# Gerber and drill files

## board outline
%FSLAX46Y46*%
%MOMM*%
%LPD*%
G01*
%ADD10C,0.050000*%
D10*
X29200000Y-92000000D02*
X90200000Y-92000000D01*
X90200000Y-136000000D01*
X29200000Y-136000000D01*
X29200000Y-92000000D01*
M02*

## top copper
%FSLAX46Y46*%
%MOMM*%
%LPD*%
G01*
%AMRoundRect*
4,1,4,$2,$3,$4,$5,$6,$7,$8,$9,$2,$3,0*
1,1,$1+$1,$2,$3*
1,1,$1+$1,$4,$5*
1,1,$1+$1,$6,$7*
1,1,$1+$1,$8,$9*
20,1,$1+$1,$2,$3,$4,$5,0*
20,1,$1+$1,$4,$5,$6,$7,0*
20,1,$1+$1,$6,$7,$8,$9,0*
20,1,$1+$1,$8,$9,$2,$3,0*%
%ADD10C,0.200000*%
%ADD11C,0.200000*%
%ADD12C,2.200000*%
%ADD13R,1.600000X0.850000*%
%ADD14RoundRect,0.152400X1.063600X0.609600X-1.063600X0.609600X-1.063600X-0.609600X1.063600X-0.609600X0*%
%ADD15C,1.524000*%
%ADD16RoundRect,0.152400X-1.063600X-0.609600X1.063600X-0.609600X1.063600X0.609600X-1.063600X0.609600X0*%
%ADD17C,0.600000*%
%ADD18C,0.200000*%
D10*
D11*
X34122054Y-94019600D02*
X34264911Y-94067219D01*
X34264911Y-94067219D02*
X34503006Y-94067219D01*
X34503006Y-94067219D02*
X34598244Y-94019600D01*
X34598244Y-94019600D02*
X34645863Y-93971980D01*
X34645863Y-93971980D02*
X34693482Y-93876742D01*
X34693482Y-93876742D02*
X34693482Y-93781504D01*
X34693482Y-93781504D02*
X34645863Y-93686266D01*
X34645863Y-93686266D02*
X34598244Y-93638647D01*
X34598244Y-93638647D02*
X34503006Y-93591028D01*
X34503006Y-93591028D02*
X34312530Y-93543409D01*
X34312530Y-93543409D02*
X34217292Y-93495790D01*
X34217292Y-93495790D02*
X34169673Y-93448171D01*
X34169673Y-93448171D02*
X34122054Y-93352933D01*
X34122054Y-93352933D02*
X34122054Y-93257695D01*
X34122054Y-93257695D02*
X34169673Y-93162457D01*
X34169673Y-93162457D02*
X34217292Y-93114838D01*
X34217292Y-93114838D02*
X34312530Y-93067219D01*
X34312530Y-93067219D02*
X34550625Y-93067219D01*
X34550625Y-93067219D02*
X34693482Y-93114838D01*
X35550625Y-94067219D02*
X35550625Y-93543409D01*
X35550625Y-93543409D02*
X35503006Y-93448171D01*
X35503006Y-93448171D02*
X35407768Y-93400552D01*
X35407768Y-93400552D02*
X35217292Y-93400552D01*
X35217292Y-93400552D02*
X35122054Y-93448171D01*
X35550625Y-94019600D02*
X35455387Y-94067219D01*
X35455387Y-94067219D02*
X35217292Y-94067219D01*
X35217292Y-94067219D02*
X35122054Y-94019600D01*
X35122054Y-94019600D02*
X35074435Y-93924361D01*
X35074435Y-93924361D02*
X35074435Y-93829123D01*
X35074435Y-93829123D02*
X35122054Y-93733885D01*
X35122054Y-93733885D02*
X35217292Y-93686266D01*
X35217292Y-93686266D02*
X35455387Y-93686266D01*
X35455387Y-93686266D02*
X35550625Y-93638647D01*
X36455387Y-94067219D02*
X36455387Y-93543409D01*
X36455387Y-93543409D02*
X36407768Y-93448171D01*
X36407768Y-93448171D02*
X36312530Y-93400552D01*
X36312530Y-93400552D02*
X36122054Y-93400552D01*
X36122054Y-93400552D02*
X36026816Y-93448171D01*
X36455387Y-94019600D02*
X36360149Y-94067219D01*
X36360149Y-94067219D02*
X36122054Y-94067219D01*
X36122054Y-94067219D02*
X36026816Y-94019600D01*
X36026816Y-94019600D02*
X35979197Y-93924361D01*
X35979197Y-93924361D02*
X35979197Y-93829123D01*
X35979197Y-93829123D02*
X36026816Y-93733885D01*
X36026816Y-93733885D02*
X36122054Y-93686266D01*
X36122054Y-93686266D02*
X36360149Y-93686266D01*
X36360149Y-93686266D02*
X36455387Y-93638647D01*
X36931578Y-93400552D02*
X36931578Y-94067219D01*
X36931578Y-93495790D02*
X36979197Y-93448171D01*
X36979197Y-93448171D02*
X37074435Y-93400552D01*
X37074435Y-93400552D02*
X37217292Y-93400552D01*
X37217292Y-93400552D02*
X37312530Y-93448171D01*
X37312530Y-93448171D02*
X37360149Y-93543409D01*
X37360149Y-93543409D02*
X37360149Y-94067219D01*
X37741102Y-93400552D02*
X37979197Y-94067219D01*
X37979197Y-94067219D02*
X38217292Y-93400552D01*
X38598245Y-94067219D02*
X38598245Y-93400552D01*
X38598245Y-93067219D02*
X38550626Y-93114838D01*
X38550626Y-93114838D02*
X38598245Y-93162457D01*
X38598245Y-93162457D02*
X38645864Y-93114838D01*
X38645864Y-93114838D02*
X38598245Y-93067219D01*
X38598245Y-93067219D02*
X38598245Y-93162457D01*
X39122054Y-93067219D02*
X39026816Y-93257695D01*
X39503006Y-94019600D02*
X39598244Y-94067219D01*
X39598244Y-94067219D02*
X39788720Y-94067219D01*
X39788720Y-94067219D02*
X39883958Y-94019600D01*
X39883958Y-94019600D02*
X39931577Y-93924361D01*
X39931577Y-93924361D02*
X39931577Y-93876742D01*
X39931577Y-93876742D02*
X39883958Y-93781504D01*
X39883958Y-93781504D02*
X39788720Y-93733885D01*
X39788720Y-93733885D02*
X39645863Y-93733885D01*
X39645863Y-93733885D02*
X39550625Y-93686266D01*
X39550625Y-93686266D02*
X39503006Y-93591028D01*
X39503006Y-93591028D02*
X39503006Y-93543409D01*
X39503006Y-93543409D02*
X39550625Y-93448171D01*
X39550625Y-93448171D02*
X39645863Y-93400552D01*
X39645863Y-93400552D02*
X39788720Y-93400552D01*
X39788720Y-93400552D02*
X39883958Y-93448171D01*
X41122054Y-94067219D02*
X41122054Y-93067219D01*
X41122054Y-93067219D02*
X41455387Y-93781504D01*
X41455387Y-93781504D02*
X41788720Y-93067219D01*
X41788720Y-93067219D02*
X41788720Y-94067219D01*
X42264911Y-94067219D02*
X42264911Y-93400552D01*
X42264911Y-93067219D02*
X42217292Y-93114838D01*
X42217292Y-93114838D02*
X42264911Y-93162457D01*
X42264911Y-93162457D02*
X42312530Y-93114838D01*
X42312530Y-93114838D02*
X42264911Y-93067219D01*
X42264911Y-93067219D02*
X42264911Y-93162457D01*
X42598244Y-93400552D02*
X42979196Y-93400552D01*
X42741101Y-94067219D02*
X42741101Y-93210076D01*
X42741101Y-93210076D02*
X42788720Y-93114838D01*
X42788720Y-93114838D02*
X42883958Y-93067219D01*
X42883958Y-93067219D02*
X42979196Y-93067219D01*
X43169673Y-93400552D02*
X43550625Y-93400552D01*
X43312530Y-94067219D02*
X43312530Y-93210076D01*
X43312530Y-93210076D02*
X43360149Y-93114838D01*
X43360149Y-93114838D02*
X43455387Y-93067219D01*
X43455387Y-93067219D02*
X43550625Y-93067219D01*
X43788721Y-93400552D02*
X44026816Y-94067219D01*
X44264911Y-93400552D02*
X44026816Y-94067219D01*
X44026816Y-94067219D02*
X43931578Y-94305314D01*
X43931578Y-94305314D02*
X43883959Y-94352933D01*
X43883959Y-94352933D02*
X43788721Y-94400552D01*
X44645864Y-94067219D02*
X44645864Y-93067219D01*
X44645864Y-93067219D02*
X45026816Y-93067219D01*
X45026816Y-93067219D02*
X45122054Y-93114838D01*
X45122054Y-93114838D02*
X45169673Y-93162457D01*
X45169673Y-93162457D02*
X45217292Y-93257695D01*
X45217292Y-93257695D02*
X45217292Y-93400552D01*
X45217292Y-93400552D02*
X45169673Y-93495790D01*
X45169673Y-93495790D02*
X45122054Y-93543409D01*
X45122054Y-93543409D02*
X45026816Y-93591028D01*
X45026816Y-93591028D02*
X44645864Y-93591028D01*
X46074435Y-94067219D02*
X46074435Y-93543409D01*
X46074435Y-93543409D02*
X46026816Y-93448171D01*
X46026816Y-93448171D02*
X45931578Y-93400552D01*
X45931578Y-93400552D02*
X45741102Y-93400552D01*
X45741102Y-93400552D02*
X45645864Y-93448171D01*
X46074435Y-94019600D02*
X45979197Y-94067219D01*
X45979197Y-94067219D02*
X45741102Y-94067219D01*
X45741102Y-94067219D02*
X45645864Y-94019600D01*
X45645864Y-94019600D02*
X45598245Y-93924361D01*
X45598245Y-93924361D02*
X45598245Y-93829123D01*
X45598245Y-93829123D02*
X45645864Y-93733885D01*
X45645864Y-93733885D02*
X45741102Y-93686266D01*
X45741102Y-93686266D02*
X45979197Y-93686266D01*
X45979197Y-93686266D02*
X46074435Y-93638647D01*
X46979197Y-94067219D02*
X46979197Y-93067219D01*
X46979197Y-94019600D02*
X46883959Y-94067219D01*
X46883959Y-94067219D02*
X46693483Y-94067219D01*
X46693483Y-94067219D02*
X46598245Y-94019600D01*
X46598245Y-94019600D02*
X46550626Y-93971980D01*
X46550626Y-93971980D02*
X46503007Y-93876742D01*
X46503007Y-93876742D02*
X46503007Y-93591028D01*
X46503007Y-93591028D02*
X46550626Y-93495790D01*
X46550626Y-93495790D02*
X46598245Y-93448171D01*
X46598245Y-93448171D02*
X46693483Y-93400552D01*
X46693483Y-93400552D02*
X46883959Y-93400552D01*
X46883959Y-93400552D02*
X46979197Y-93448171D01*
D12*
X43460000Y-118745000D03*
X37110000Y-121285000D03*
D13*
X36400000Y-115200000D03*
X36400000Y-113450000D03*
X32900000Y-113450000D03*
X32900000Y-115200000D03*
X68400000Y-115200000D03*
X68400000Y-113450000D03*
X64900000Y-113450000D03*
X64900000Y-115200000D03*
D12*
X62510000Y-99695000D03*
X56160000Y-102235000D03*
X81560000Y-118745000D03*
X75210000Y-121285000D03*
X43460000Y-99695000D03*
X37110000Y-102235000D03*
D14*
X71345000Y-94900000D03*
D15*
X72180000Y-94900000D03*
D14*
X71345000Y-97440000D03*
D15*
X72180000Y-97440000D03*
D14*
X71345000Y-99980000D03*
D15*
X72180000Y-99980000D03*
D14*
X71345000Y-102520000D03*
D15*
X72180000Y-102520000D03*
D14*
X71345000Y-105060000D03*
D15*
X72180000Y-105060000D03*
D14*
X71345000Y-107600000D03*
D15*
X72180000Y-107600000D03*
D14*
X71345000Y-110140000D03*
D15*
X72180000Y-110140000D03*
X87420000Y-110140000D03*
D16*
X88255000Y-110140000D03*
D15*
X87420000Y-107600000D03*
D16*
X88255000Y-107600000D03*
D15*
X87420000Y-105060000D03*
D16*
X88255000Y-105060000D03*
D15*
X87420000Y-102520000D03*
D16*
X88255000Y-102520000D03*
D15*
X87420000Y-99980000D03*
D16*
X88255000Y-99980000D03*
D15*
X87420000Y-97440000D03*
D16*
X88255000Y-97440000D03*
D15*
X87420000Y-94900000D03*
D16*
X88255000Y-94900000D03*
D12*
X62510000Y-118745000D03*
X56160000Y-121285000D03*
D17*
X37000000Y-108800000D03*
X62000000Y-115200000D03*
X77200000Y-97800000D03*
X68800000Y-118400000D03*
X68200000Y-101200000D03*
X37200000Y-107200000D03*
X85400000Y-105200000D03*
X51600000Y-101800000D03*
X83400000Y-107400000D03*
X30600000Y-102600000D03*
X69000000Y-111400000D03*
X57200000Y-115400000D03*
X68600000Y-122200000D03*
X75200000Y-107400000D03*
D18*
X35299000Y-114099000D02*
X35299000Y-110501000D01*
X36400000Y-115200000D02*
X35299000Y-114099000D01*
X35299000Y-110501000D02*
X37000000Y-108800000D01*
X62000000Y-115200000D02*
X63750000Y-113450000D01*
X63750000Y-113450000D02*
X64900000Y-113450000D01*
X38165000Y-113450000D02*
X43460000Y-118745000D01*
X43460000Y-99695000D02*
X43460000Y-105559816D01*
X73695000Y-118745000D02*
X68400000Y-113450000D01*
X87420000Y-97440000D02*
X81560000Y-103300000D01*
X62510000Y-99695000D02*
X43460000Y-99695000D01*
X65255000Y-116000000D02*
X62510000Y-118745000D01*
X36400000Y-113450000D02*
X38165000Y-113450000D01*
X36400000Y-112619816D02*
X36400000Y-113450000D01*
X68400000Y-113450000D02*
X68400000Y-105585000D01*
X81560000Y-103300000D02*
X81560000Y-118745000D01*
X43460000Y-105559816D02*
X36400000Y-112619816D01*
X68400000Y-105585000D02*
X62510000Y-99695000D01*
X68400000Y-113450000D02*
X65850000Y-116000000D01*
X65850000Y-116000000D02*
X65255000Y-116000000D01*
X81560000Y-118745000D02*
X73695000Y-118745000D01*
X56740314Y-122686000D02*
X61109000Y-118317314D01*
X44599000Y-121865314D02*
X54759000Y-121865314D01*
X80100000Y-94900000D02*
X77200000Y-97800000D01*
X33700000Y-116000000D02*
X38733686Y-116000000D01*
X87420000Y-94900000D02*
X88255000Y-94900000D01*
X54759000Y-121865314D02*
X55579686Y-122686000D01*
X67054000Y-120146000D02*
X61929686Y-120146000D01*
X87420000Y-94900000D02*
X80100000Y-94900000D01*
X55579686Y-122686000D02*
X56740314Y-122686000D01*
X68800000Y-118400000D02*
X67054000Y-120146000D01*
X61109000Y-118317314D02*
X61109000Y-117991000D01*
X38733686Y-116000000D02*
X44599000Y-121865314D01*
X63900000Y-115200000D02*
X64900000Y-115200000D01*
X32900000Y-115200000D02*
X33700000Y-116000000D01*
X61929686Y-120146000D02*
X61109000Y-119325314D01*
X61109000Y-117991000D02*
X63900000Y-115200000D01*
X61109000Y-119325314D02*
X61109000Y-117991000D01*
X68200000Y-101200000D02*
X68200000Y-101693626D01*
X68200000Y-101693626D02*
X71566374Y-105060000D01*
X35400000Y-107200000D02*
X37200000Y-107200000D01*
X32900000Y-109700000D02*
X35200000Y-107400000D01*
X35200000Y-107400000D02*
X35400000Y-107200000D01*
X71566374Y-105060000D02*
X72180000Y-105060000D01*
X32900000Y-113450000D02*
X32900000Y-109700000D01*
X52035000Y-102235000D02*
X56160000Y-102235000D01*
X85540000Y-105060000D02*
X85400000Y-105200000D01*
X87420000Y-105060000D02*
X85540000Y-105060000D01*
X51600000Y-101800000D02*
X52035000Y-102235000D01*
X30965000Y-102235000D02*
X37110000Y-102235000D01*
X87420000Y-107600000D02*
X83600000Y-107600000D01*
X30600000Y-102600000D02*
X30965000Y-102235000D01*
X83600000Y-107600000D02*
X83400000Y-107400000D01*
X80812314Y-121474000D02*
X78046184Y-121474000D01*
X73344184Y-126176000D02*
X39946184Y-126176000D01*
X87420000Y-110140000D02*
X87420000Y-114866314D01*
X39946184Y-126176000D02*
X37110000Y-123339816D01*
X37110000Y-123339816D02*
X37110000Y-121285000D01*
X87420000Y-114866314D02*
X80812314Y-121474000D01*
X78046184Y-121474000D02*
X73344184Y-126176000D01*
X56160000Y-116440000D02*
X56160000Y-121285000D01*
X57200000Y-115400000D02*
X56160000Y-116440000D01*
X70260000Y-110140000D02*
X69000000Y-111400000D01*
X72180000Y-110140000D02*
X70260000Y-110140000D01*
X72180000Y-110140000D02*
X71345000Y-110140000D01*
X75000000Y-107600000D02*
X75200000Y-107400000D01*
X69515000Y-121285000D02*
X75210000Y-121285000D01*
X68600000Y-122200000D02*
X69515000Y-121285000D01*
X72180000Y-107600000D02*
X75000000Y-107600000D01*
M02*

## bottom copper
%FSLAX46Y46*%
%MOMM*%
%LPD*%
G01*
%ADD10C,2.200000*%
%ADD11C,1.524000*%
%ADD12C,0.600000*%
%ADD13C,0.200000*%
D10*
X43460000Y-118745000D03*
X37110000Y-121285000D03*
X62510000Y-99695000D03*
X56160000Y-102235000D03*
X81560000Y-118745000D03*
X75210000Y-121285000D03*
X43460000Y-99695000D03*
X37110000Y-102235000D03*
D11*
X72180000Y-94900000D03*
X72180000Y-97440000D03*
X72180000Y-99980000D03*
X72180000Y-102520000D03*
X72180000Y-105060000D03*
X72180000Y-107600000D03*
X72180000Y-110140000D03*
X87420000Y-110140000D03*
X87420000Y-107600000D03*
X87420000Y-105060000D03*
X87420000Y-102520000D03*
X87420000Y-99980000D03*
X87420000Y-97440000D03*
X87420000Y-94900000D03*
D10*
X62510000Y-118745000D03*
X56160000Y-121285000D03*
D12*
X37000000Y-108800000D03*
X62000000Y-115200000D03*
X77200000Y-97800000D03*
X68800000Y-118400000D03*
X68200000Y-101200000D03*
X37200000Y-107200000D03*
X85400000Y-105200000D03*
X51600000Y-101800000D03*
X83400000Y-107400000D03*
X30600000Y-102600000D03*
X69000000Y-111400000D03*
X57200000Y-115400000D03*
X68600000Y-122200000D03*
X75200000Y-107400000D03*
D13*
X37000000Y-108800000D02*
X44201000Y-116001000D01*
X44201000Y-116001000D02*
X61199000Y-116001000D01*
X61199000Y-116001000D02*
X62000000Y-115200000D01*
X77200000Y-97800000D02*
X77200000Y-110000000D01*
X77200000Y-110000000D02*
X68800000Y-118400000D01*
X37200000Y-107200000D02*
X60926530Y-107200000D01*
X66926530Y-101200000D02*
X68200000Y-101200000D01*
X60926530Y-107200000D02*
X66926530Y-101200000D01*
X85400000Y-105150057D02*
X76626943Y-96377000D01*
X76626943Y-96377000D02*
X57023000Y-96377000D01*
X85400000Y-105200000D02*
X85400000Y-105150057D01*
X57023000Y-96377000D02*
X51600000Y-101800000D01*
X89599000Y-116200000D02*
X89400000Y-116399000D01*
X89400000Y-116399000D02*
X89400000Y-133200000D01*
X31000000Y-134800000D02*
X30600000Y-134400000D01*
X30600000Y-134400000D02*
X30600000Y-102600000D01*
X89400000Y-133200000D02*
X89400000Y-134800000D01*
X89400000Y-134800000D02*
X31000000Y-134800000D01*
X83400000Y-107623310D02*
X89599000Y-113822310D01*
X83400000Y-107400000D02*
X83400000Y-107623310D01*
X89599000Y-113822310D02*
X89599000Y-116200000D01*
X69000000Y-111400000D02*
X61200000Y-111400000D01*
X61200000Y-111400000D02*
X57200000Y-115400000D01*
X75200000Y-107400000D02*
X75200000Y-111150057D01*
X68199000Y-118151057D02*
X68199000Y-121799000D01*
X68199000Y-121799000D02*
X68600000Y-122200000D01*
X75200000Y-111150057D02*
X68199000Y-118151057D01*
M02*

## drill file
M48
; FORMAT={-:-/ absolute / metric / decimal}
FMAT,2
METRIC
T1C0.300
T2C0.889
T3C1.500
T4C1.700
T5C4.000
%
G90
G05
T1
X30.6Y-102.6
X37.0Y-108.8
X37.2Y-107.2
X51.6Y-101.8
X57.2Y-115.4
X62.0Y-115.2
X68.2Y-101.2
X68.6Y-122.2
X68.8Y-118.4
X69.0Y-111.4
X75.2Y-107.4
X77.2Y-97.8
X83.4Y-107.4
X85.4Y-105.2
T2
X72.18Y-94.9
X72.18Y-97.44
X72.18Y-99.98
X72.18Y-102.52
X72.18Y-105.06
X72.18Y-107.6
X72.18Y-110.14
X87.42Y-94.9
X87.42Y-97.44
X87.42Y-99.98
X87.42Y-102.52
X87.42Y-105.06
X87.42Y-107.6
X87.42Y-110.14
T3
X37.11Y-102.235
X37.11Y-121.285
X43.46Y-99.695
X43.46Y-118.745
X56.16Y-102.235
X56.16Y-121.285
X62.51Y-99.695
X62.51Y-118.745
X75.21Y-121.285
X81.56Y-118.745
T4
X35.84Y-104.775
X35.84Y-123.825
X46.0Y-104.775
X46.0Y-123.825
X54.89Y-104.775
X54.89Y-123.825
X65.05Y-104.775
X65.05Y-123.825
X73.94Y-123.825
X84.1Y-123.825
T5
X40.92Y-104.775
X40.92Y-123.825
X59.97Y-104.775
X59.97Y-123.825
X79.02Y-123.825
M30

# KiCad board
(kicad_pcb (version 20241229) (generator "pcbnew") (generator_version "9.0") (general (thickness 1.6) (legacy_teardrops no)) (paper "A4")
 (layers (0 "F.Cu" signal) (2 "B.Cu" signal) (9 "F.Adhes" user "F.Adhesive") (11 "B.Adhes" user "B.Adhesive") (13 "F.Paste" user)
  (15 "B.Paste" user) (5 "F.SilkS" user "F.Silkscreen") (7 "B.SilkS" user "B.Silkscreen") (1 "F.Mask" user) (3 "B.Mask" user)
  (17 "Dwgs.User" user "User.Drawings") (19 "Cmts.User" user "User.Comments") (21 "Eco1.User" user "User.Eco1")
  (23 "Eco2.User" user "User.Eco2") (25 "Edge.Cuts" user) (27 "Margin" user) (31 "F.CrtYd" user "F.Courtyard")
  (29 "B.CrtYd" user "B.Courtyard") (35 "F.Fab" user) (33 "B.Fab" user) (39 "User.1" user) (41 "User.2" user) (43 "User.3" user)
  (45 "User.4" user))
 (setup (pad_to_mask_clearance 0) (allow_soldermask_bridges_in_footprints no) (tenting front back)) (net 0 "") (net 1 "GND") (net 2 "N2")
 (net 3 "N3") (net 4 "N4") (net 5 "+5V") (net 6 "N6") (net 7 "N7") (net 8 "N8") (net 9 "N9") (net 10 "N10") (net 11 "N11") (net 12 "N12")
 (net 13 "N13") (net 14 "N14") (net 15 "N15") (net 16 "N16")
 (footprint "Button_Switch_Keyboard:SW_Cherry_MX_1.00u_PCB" (layer "F.Cu") (at 43.46 118.745)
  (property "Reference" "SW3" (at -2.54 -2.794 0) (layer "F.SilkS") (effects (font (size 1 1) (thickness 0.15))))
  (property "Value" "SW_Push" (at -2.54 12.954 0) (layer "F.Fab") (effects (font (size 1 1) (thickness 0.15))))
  (pad "" np_thru_hole circle (at -7.62 5.08) (size 1.7 1.7) (drill 1.7) (layers "*.Cu" "*.Mask"))
  (pad "" np_thru_hole circle (at -2.54 5.08) (size 4 4) (drill 4) (layers "*.Cu" "*.Mask"))
  (pad "" np_thru_hole circle (at 2.54 5.08) (size 1.7 1.7) (drill 1.7) (layers "*.Cu" "*.Mask"))
  (pad "1" thru_hole circle (at 0 0) (size 2.2 2.2) (drill 1.5) (layers "*.Cu" "*.Mask") (remove_unused_layers no) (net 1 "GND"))
  (pad "2" thru_hole circle (at -6.35 2.54) (size 2.2 2.2) (drill 1.5) (layers "*.Cu" "*.Mask") (remove_unused_layers no) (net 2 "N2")))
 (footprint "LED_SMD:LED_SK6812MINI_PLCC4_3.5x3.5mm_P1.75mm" (layer "F.Cu") (at 34.65 114.325 180)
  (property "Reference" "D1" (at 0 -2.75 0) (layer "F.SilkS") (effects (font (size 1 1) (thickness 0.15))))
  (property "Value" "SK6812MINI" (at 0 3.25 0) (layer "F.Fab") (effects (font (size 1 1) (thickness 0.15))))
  (pad "1" smd rect (at -1.75 -0.875 180) (size 1.6 0.85) (layers "F.Cu" "F.Mask" "F.Paste") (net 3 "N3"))
  (pad "2" smd rect (at -1.75 0.875 180) (size 1.6 0.85) (layers "F.Cu" "F.Mask" "F.Paste") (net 1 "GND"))
  (pad "3" smd rect (at 1.75 0.875 180) (size 1.6 0.85) (layers "F.Cu" "F.Mask" "F.Paste") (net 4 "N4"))
  (pad "4" smd rect (at 1.75 -0.875 180) (size 1.6 0.85) (layers "F.Cu" "F.Mask" "F.Paste") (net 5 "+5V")))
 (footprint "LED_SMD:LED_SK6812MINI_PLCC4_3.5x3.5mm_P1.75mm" (layer "F.Cu") (at 66.65 114.325 180)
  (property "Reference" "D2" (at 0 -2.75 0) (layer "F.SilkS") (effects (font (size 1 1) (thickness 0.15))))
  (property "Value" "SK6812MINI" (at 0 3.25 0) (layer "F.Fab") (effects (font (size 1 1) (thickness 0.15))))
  (pad "1" smd rect (at -1.75 -0.875 180) (size 1.6 0.85) (layers "F.Cu" "F.Mask" "F.Paste") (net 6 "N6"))
  (pad "2" smd rect (at -1.75 0.875 180) (size 1.6 0.85) (layers "F.Cu" "F.Mask" "F.Paste") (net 1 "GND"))
  (pad "3" smd rect (at 1.75 0.875 180) (size 1.6 0.85) (layers "F.Cu" "F.Mask" "F.Paste") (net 3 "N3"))
  (pad "4" smd rect (at 1.75 -0.875 180) (size 1.6 0.85) (layers "F.Cu" "F.Mask" "F.Paste") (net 5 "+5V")))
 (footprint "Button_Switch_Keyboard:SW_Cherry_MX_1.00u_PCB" (layer "F.Cu") (at 62.51 99.695)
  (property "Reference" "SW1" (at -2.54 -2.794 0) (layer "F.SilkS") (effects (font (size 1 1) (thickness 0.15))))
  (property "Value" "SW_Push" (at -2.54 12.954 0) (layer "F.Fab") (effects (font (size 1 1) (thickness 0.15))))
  (pad "" np_thru_hole circle (at -7.62 5.08) (size 1.7 1.7) (drill 1.7) (layers "*.Cu" "*.Mask"))
  (pad "" np_thru_hole circle (at -2.54 5.08) (size 4 4) (drill 4) (layers "*.Cu" "*.Mask"))
  (pad "" np_thru_hole circle (at 2.54 5.08) (size 1.7 1.7) (drill 1.7) (layers "*.Cu" "*.Mask"))
  (pad "1" thru_hole circle (at 0 0) (size 2.2 2.2) (drill 1.5) (layers "*.Cu" "*.Mask") (remove_unused_layers no) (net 1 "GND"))
  (pad "2" thru_hole circle (at -6.35 2.54) (size 2.2 2.2) (drill 1.5) (layers "*.Cu" "*.Mask") (remove_unused_layers no) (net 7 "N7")))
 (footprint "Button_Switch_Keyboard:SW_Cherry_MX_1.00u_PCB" (layer "F.Cu") (at 81.56 118.745)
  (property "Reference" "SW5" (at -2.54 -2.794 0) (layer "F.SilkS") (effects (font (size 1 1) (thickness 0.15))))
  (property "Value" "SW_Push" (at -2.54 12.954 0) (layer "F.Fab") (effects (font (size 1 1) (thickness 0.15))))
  (pad "" np_thru_hole circle (at -7.62 5.08) (size 1.7 1.7) (drill 1.7) (layers "*.Cu" "*.Mask"))
  (pad "" np_thru_hole circle (at -2.54 5.08) (size 4 4) (drill 4) (layers "*.Cu" "*.Mask"))
  (pad "" np_thru_hole circle (at 2.54 5.08) (size 1.7 1.7) (drill 1.7) (layers "*.Cu" "*.Mask"))
  (pad "1" thru_hole circle (at 0 0) (size 2.2 2.2) (drill 1.5) (layers "*.Cu" "*.Mask") (remove_unused_layers no) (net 1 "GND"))
  (pad "2" thru_hole circle (at -6.35 2.54) (size 2.2 2.2) (drill 1.5) (layers "*.Cu" "*.Mask") (remove_unused_layers no) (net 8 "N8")))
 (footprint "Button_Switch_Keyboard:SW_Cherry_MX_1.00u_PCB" (layer "F.Cu") (at 43.46 99.695)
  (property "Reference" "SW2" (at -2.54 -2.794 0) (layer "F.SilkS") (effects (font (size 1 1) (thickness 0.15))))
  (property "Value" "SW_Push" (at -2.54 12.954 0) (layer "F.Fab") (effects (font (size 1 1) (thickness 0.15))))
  (pad "" np_thru_hole circle (at -7.62 5.08) (size 1.7 1.7) (drill 1.7) (layers "*.Cu" "*.Mask"))
  (pad "" np_thru_hole circle (at -2.54 5.08) (size 4 4) (drill 4) (layers "*.Cu" "*.Mask"))
  (pad "" np_thru_hole circle (at 2.54 5.08) (size 1.7 1.7) (drill 1.7) (layers "*.Cu" "*.Mask"))
  (pad "1" thru_hole circle (at 0 0) (size 2.2 2.2) (drill 1.5) (layers "*.Cu" "*.Mask") (remove_unused_layers no) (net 1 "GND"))
  (pad "2" thru_hole circle (at -6.35 2.54) (size 2.2 2.2) (drill 1.5) (layers "*.Cu" "*.Mask") (remove_unused_layers no) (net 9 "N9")))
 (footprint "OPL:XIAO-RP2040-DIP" (layer "F.Cu") (at 79.8 102.52)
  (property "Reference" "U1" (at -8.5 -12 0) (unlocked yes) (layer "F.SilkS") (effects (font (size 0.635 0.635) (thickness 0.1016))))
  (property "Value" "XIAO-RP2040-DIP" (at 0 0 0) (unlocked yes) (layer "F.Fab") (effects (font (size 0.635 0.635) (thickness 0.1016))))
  (pad "1" smd roundrect (at -8.455 -7.62 180) (size 2.432 1.524) (layers "F.Cu" "F.Mask") (roundrect_rratio 0.1) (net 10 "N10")
   (thermal_bridge_angle 45))
  (pad "1" thru_hole circle (at -7.62 -7.62 180) (size 1.524 1.524) (drill 0.889) (layers "*.Cu" "*.Mask") (remove_unused_layers no)
   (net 10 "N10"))
  (pad "2" smd roundrect (at -8.455 -5.08 180) (size 2.432 1.524) (layers "F.Cu" "F.Mask") (roundrect_rratio 0.1) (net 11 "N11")
   (thermal_bridge_angle 45))
  (pad "2" thru_hole circle (at -7.62 -5.08 180) (size 1.524 1.524) (drill 0.889) (layers "*.Cu" "*.Mask") (remove_unused_layers no)
   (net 11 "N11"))
  (pad "3" smd roundrect (at -8.455 -2.54 180) (size 2.432 1.524) (layers "F.Cu" "F.Mask") (roundrect_rratio 0.1) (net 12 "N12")
   (thermal_bridge_angle 45))
  (pad "3" thru_hole circle (at -7.62 -2.54 180) (size 1.524 1.524) (drill 0.889) (layers "*.Cu" "*.Mask") (remove_unused_layers no)
   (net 12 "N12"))
  (pad "4" smd roundrect (at -8.455 0 180) (size 2.432 1.524) (layers "F.Cu" "F.Mask") (roundrect_rratio 0.1) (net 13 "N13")
   (thermal_bridge_angle 45))
  (pad "4" thru_hole circle (at -7.62 0 180) (size 1.524 1.524) (drill 0.889) (layers "*.Cu" "*.Mask") (remove_unused_layers no)
   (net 13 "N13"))
  (pad "5" smd roundrect (at -8.455 2.54 180) (size 2.432 1.524) (layers "F.Cu" "F.Mask") (roundrect_rratio 0.1) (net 4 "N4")
   (thermal_bridge_angle 45))
  (pad "5" thru_hole circle (at -7.62 2.54 180) (size 1.524 1.524) (drill 0.889) (layers "*.Cu" "*.Mask") (remove_unused_layers no)
   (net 4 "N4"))
  (pad "6" smd roundrect (at -8.455 5.08 180) (size 2.432 1.524) (layers "F.Cu" "F.Mask") (roundrect_rratio 0.1) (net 8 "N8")
   (thermal_bridge_angle 45))
  (pad "6" thru_hole circle (at -7.62 5.08 180) (size 1.524 1.524) (drill 0.889) (layers "*.Cu" "*.Mask") (remove_unused_layers no)
   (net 8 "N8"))
  (pad "7" smd roundrect (at -8.455 7.62 180) (size 2.432 1.524) (layers "F.Cu" "F.Mask") (roundrect_rratio 0.1) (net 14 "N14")
   (thermal_bridge_angle 45))
  (pad "7" thru_hole circle (at -7.62 7.62 180) (size 1.524 1.524) (drill 0.889) (layers "*.Cu" "*.Mask") (remove_unused_layers no)
   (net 14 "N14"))
  (pad "8" thru_hole circle (at 7.62 7.62) (size 1.524 1.524) (drill 0.889) (layers "*.Cu" "*.Mask") (remove_unused_layers no) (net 2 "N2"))
  (pad "8" smd roundrect (at 8.455 7.62) (size 2.432 1.524) (layers "F.Cu" "F.Mask") (roundrect_rratio 0.1) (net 2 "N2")
   (thermal_bridge_angle 45))
  (pad "9" thru_hole circle (at 7.62 5.08) (size 1.524 1.524) (drill 0.889) (layers "*.Cu" "*.Mask") (remove_unused_layers no) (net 9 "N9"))
  (pad "9" smd roundrect (at 8.455 5.08) (size 2.432 1.524) (layers "F.Cu" "F.Mask") (roundrect_rratio 0.1) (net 9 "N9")
   (thermal_bridge_angle 45))
  (pad "10" thru_hole circle (at 7.62 2.54) (size 1.524 1.524) (drill 0.889) (layers "*.Cu" "*.Mask") (remove_unused_layers no) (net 7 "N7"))
  (pad "10" smd roundrect (at 8.455 2.54) (size 2.432 1.524) (layers "F.Cu" "F.Mask") (roundrect_rratio 0.1) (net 7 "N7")
   (thermal_bridge_angle 45))
  (pad "11" thru_hole circle (at 7.62 0) (size 1.524 1.524) (drill 0.889) (layers "*.Cu" "*.Mask") (remove_unused_layers no) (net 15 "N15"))
  (pad "11" smd roundrect (at 8.455 0) (size 2.432 1.524) (layers "F.Cu" "F.Mask") (roundrect_rratio 0.1) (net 15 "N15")
   (thermal_bridge_angle 45))
  (pad "12" thru_hole circle (at 7.62 -2.54) (size 1.524 1.524) (drill 0.889) (layers "*.Cu" "*.Mask") (remove_unused_layers no)
   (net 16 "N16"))
  (pad "12" smd roundrect (at 8.455 -2.54) (size 2.432 1.524) (layers "F.Cu" "F.Mask") (roundrect_rratio 0.1) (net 16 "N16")
   (thermal_bridge_angle 45))
  (pad "13" thru_hole circle (at 7.62 -5.08) (size 1.524 1.524) (drill 0.889) (layers "*.Cu" "*.Mask") (remove_unused_layers no)
   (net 1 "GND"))
  (pad "13" smd roundrect (at 8.455 -5.08) (size 2.432 1.524) (layers "F.Cu" "F.Mask") (roundrect_rratio 0.1) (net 1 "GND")
   (thermal_bridge_angle 45))
  (pad "14" thru_hole circle (at 7.62 -7.62) (size 1.524 1.524) (drill 0.889) (layers "*.Cu" "*.Mask") (remove_unused_layers no)
   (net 5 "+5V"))
  (pad "14" smd roundrect (at 8.455 -7.62) (size 2.432 1.524) (layers "F.Cu" "F.Mask") (roundrect_rratio 0.1) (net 5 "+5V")
   (thermal_bridge_angle 45)))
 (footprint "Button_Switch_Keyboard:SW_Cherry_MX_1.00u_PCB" (layer "F.Cu") (at 62.51 118.745)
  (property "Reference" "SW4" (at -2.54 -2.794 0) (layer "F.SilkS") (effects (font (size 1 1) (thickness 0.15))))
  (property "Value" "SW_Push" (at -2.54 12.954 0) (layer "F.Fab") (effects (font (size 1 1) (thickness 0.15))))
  (pad "" np_thru_hole circle (at -7.62 5.08) (size 1.7 1.7) (drill 1.7) (layers "*.Cu" "*.Mask"))
  (pad "" np_thru_hole circle (at -2.54 5.08) (size 4 4) (drill 4) (layers "*.Cu" "*.Mask"))
  (pad "" np_thru_hole circle (at 2.54 5.08) (size 1.7 1.7) (drill 1.7) (layers "*.Cu" "*.Mask"))
  (pad "1" thru_hole circle (at 0 0) (size 2.2 2.2) (drill 1.5) (layers "*.Cu" "*.Mask") (remove_unused_layers no) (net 1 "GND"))
  (pad "2" thru_hole circle (at -6.35 2.54) (size 2.2 2.2) (drill 1.5) (layers "*.Cu" "*.Mask") (remove_unused_layers no) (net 14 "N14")))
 (gr_rect (start 29.2 92) (end 90.2 136) (stroke (width 0.05) (type default)) (fill no) (layer "Edge.Cuts"))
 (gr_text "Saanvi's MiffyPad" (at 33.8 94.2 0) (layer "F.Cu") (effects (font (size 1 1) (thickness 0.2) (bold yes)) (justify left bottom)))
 (segment (start 35.299 114.099) (end 35.299 110.501) (width 0.2) (layer "F.Cu") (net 3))
 (segment (start 36.4 115.2) (end 35.299 114.099) (width 0.2) (layer "F.Cu") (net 3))
 (segment (start 35.299 110.501) (end 37 108.8) (width 0.2) (layer "F.Cu") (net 3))
 (segment (start 62 115.2) (end 63.75 113.45) (width 0.2) (layer "F.Cu") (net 3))
 (segment (start 63.75 113.45) (end 64.9 113.45) (width 0.2) (layer "F.Cu") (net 3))
 (via (at 37 108.8) (size 0.6) (drill 0.3) (layers "F.Cu" "B.Cu") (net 3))
 (via (at 62 115.2) (size 0.6) (drill 0.3) (layers "F.Cu" "B.Cu") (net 3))
 (segment (start 37 108.8) (end 44.201 116.001) (width 0.2) (layer "B.Cu") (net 3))
 (segment (start 44.201 116.001) (end 61.199 116.001) (width 0.2) (layer "B.Cu") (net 3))
 (segment (start 61.199 116.001) (end 62 115.2) (width 0.2) (layer "B.Cu") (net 3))
 (segment (start 38.165 113.45) (end 43.46 118.745) (width 0.2) (layer "F.Cu") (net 1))
 (segment (start 43.46 99.695) (end 43.46 105.559816) (width 0.2) (layer "F.Cu") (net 1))
 (segment (start 73.695 118.745) (end 68.4 113.45) (width 0.2) (layer "F.Cu") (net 1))
 (segment (start 87.42 97.44) (end 81.56 103.3) (width 0.2) (layer "F.Cu") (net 1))
 (segment (start 62.51 99.695) (end 43.46 99.695) (width 0.2) (layer "F.Cu") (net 1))
 (segment (start 65.255 116) (end 62.51 118.745) (width 0.2) (layer "F.Cu") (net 1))
 (segment (start 36.4 113.45) (end 38.165 113.45) (width 0.2) (layer "F.Cu") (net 1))
 (segment (start 36.4 112.619816) (end 36.4 113.45) (width 0.2) (layer "F.Cu") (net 1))
 (segment (start 68.4 113.45) (end 68.4 105.585) (width 0.2) (layer "F.Cu") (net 1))
 (segment (start 81.56 103.3) (end 81.56 118.745) (width 0.2) (layer "F.Cu") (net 1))
 (segment (start 43.46 105.559816) (end 36.4 112.619816) (width 0.2) (layer "F.Cu") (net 1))
 (segment (start 68.4 105.585) (end 62.51 99.695) (width 0.2) (layer "F.Cu") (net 1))
 (segment (start 68.4 113.45) (end 65.85 116) (width 0.2) (layer "F.Cu") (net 1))
 (segment (start 65.85 116) (end 65.255 116) (width 0.2) (layer "F.Cu") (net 1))
 (segment (start 81.56 118.745) (end 73.695 118.745) (width 0.2) (layer "F.Cu") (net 1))
 (segment (start 56.740314 122.686) (end 61.109 118.317314) (width 0.2) (layer "F.Cu") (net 5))
 (segment (start 44.599 121.865314) (end 54.759 121.865314) (width 0.2) (layer "F.Cu") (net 5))
 (segment (start 80.1 94.9) (end 77.2 97.8) (width 0.2) (layer "F.Cu") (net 5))
 (segment (start 33.7 116) (end 38.733686 116) (width 0.2) (layer "F.Cu") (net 5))
 (segment (start 87.42 94.9) (end 88.255 94.9) (width 0.2) (layer "F.Cu") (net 5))
 (segment (start 54.759 121.865314) (end 55.579686 122.686) (width 0.2) (layer "F.Cu") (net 5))
 (segment (start 67.054 120.146) (end 61.929686 120.146) (width 0.2) (layer "F.Cu") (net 5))
 (segment (start 87.42 94.9) (end 80.1 94.9) (width 0.2) (layer "F.Cu") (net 5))
 (segment (start 55.579686 122.686) (end 56.740314 122.686) (width 0.2) (layer "F.Cu") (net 5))
 (segment (start 68.8 118.4) (end 67.054 120.146) (width 0.2) (layer "F.Cu") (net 5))
 (segment (start 61.109 118.317314) (end 61.109 117.991) (width 0.2) (layer "F.Cu") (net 5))
 (segment (start 38.733686 116) (end 44.599 121.865314) (width 0.2) (layer "F.Cu") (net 5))
 (segment (start 63.9 115.2) (end 64.9 115.2) (width 0.2) (layer "F.Cu") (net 5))
 (segment (start 32.9 115.2) (end 33.7 116) (width 0.2) (layer "F.Cu") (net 5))
 (segment (start 61.929686 120.146) (end 61.109 119.325314) (width 0.2) (layer "F.Cu") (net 5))
 (segment (start 61.109 117.991) (end 63.9 115.2) (width 0.2) (layer "F.Cu") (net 5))
 (segment (start 61.109 119.325314) (end 61.109 117.991) (width 0.2) (layer "F.Cu") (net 5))
 (via (at 77.2 97.8) (size 0.6) (drill 0.3) (layers "F.Cu" "B.Cu") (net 5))
 (via (at 68.8 118.4) (size 0.6) (drill 0.3) (layers "F.Cu" "B.Cu") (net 5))
 (segment (start 77.2 97.8) (end 77.2 110) (width 0.2) (layer "B.Cu") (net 5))
 (segment (start 77.2 110) (end 68.8 118.4) (width 0.2) (layer "B.Cu") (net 5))
 (segment (start 68.2 101.2) (end 68.2 101.693626) (width 0.2) (layer "F.Cu") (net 4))
 (segment (start 68.2 101.693626) (end 71.566374 105.06) (width 0.2) (layer "F.Cu") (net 4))
 (segment (start 35.4 107.2) (end 37.2 107.2) (width 0.2) (layer "F.Cu") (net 4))
 (segment (start 32.9 109.7) (end 35.2 107.4) (width 0.2) (layer "F.Cu") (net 4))
 (segment (start 35.2 107.4) (end 35.4 107.2) (width 0.2) (layer "F.Cu") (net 4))
 (segment (start 71.566374 105.06) (end 72.18 105.06) (width 0.2) (layer "F.Cu") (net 4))
 (segment (start 32.9 113.45) (end 32.9 109.7) (width 0.2) (layer "F.Cu") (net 4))
 (via (at 68.2 101.2) (size 0.6) (drill 0.3) (layers "F.Cu" "B.Cu") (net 4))
 (via (at 37.2 107.2) (size 0.6) (drill 0.3) (layers "F.Cu" "B.Cu") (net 4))
 (segment (start 37.2 107.2) (end 60.92653 107.2) (width 0.2) (layer "B.Cu") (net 4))
 (segment (start 66.92653 101.2) (end 68.2 101.2) (width 0.2) (layer "B.Cu") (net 4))
 (segment (start 60.92653 107.2) (end 66.92653 101.2) (width 0.2) (layer "B.Cu") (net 4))
 (segment (start 52.035 102.235) (end 56.16 102.235) (width 0.2) (layer "F.Cu") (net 7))
 (segment (start 85.54 105.06) (end 85.4 105.2) (width 0.2) (layer "F.Cu") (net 7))
 (segment (start 87.42 105.06) (end 85.54 105.06) (width 0.2) (layer "F.Cu") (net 7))
 (segment (start 51.6 101.8) (end 52.035 102.235) (width 0.2) (layer "F.Cu") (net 7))
 (via (at 85.4 105.2) (size 0.6) (drill 0.3) (layers "F.Cu" "B.Cu") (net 7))
 (via (at 51.6 101.8) (size 0.6) (drill 0.3) (layers "F.Cu" "B.Cu") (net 7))
 (segment (start 85.4 105.150057) (end 76.626943 96.377) (width 0.2) (layer "B.Cu") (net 7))
 (segment (start 76.626943 96.377) (end 57.023 96.377) (width 0.2) (layer "B.Cu") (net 7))
 (segment (start 85.4 105.2) (end 85.4 105.150057) (width 0.2) (layer "B.Cu") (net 7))
 (segment (start 57.023 96.377) (end 51.6 101.8) (width 0.2) (layer "B.Cu") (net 7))
 (segment (start 30.965 102.235) (end 37.11 102.235) (width 0.2) (layer "F.Cu") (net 9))
 (segment (start 87.42 107.6) (end 83.6 107.6) (width 0.2) (layer "F.Cu") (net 9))
 (segment (start 30.6 102.6) (end 30.965 102.235) (width 0.2) (layer "F.Cu") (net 9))
 (segment (start 83.6 107.6) (end 83.4 107.4) (width 0.2) (layer "F.Cu") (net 9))
 (via (at 83.4 107.4) (size 0.6) (drill 0.3) (layers "F.Cu" "B.Cu") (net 9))
 (via (at 30.6 102.6) (size 0.6) (drill 0.3) (layers "F.Cu" "B.Cu") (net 9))
 (segment (start 89.599 116.2) (end 89.4 116.399) (width 0.2) (layer "B.Cu") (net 9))
 (segment (start 89.4 116.399) (end 89.4 133.2) (width 0.2) (layer "B.Cu") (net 9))
 (segment (start 31 134.8) (end 30.6 134.4) (width 0.2) (layer "B.Cu") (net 9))
 (segment (start 30.6 134.4) (end 30.6 102.6) (width 0.2) (layer "B.Cu") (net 9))
 (segment (start 89.4 133.2) (end 89.4 134.8) (width 0.2) (layer "B.Cu") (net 9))
 (segment (start 89.4 134.8) (end 31 134.8) (width 0.2) (layer "B.Cu") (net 9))
 (segment (start 83.4 107.62331) (end 89.599 113.82231) (width 0.2) (layer "B.Cu") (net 9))
 (segment (start 83.4 107.4) (end 83.4 107.62331) (width 0.2) (layer "B.Cu") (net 9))
 (segment (start 89.599 113.82231) (end 89.599 116.2) (width 0.2) (layer "B.Cu") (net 9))
 (segment (start 80.812314 121.474) (end 78.046184 121.474) (width 0.2) (layer "F.Cu") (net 2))
 (segment (start 73.344184 126.176) (end 39.946184 126.176) (width 0.2) (layer "F.Cu") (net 2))
 (segment (start 87.42 110.14) (end 87.42 114.866314) (width 0.2) (layer "F.Cu") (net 2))
 (segment (start 39.946184 126.176) (end 37.11 123.339816) (width 0.2) (layer "F.Cu") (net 2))
 (segment (start 37.11 123.339816) (end 37.11 121.285) (width 0.2) (layer "F.Cu") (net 2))
 (segment (start 87.42 114.866314) (end 80.812314 121.474) (width 0.2) (layer "F.Cu") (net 2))
 (segment (start 78.046184 121.474) (end 73.344184 126.176) (width 0.2) (layer "F.Cu") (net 2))
 (segment (start 56.16 116.44) (end 56.16 121.285) (width 0.2) (layer "F.Cu") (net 14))
 (segment (start 57.2 115.4) (end 56.16 116.44) (width 0.2) (layer "F.Cu") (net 14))
 (segment (start 70.26 110.14) (end 69 111.4) (width 0.2) (layer "F.Cu") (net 14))
 (segment (start 72.18 110.14) (end 70.26 110.14) (width 0.2) (layer "F.Cu") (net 14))
 (segment (start 72.18 110.14) (end 71.345 110.14) (width 0.2) (layer "F.Cu") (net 14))
 (via (at 69 111.4) (size 0.6) (drill 0.3) (layers "F.Cu" "B.Cu") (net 14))
 (via (at 57.2 115.4) (size 0.6) (drill 0.3) (layers "F.Cu" "B.Cu") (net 14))
 (segment (start 69 111.4) (end 61.2 111.4) (width 0.2) (layer "B.Cu") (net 14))
 (segment (start 61.2 111.4) (end 57.2 115.4) (width 0.2) (layer "B.Cu") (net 14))
 (segment (start 75 107.6) (end 75.2 107.4) (width 0.2) (layer "F.Cu") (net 8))
 (segment (start 69.515 121.285) (end 75.21 121.285) (width 0.2) (layer "F.Cu") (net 8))
 (segment (start 68.6 122.2) (end 69.515 121.285) (width 0.2) (layer "F.Cu") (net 8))
 (segment (start 72.18 107.6) (end 75 107.6) (width 0.2) (layer "F.Cu") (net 8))
 (via (at 68.6 122.2) (size 0.6) (drill 0.3) (layers "F.Cu" "B.Cu") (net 8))
 (via (at 75.2 107.4) (size 0.6) (drill 0.3) (layers "F.Cu" "B.Cu") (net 8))
 (segment (start 75.2 107.4) (end 75.2 111.150057) (width 0.2) (layer "B.Cu") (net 8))
 (segment (start 68.199 118.151057) (end 68.199 121.799) (width 0.2) (layer "B.Cu") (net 8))
 (segment (start 68.199 121.799) (end 68.6 122.2) (width 0.2) (layer "B.Cu") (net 8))
 (segment (start 75.2 111.150057) (end 68.199 118.151057) (width 0.2) (layer "B.Cu") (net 8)))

